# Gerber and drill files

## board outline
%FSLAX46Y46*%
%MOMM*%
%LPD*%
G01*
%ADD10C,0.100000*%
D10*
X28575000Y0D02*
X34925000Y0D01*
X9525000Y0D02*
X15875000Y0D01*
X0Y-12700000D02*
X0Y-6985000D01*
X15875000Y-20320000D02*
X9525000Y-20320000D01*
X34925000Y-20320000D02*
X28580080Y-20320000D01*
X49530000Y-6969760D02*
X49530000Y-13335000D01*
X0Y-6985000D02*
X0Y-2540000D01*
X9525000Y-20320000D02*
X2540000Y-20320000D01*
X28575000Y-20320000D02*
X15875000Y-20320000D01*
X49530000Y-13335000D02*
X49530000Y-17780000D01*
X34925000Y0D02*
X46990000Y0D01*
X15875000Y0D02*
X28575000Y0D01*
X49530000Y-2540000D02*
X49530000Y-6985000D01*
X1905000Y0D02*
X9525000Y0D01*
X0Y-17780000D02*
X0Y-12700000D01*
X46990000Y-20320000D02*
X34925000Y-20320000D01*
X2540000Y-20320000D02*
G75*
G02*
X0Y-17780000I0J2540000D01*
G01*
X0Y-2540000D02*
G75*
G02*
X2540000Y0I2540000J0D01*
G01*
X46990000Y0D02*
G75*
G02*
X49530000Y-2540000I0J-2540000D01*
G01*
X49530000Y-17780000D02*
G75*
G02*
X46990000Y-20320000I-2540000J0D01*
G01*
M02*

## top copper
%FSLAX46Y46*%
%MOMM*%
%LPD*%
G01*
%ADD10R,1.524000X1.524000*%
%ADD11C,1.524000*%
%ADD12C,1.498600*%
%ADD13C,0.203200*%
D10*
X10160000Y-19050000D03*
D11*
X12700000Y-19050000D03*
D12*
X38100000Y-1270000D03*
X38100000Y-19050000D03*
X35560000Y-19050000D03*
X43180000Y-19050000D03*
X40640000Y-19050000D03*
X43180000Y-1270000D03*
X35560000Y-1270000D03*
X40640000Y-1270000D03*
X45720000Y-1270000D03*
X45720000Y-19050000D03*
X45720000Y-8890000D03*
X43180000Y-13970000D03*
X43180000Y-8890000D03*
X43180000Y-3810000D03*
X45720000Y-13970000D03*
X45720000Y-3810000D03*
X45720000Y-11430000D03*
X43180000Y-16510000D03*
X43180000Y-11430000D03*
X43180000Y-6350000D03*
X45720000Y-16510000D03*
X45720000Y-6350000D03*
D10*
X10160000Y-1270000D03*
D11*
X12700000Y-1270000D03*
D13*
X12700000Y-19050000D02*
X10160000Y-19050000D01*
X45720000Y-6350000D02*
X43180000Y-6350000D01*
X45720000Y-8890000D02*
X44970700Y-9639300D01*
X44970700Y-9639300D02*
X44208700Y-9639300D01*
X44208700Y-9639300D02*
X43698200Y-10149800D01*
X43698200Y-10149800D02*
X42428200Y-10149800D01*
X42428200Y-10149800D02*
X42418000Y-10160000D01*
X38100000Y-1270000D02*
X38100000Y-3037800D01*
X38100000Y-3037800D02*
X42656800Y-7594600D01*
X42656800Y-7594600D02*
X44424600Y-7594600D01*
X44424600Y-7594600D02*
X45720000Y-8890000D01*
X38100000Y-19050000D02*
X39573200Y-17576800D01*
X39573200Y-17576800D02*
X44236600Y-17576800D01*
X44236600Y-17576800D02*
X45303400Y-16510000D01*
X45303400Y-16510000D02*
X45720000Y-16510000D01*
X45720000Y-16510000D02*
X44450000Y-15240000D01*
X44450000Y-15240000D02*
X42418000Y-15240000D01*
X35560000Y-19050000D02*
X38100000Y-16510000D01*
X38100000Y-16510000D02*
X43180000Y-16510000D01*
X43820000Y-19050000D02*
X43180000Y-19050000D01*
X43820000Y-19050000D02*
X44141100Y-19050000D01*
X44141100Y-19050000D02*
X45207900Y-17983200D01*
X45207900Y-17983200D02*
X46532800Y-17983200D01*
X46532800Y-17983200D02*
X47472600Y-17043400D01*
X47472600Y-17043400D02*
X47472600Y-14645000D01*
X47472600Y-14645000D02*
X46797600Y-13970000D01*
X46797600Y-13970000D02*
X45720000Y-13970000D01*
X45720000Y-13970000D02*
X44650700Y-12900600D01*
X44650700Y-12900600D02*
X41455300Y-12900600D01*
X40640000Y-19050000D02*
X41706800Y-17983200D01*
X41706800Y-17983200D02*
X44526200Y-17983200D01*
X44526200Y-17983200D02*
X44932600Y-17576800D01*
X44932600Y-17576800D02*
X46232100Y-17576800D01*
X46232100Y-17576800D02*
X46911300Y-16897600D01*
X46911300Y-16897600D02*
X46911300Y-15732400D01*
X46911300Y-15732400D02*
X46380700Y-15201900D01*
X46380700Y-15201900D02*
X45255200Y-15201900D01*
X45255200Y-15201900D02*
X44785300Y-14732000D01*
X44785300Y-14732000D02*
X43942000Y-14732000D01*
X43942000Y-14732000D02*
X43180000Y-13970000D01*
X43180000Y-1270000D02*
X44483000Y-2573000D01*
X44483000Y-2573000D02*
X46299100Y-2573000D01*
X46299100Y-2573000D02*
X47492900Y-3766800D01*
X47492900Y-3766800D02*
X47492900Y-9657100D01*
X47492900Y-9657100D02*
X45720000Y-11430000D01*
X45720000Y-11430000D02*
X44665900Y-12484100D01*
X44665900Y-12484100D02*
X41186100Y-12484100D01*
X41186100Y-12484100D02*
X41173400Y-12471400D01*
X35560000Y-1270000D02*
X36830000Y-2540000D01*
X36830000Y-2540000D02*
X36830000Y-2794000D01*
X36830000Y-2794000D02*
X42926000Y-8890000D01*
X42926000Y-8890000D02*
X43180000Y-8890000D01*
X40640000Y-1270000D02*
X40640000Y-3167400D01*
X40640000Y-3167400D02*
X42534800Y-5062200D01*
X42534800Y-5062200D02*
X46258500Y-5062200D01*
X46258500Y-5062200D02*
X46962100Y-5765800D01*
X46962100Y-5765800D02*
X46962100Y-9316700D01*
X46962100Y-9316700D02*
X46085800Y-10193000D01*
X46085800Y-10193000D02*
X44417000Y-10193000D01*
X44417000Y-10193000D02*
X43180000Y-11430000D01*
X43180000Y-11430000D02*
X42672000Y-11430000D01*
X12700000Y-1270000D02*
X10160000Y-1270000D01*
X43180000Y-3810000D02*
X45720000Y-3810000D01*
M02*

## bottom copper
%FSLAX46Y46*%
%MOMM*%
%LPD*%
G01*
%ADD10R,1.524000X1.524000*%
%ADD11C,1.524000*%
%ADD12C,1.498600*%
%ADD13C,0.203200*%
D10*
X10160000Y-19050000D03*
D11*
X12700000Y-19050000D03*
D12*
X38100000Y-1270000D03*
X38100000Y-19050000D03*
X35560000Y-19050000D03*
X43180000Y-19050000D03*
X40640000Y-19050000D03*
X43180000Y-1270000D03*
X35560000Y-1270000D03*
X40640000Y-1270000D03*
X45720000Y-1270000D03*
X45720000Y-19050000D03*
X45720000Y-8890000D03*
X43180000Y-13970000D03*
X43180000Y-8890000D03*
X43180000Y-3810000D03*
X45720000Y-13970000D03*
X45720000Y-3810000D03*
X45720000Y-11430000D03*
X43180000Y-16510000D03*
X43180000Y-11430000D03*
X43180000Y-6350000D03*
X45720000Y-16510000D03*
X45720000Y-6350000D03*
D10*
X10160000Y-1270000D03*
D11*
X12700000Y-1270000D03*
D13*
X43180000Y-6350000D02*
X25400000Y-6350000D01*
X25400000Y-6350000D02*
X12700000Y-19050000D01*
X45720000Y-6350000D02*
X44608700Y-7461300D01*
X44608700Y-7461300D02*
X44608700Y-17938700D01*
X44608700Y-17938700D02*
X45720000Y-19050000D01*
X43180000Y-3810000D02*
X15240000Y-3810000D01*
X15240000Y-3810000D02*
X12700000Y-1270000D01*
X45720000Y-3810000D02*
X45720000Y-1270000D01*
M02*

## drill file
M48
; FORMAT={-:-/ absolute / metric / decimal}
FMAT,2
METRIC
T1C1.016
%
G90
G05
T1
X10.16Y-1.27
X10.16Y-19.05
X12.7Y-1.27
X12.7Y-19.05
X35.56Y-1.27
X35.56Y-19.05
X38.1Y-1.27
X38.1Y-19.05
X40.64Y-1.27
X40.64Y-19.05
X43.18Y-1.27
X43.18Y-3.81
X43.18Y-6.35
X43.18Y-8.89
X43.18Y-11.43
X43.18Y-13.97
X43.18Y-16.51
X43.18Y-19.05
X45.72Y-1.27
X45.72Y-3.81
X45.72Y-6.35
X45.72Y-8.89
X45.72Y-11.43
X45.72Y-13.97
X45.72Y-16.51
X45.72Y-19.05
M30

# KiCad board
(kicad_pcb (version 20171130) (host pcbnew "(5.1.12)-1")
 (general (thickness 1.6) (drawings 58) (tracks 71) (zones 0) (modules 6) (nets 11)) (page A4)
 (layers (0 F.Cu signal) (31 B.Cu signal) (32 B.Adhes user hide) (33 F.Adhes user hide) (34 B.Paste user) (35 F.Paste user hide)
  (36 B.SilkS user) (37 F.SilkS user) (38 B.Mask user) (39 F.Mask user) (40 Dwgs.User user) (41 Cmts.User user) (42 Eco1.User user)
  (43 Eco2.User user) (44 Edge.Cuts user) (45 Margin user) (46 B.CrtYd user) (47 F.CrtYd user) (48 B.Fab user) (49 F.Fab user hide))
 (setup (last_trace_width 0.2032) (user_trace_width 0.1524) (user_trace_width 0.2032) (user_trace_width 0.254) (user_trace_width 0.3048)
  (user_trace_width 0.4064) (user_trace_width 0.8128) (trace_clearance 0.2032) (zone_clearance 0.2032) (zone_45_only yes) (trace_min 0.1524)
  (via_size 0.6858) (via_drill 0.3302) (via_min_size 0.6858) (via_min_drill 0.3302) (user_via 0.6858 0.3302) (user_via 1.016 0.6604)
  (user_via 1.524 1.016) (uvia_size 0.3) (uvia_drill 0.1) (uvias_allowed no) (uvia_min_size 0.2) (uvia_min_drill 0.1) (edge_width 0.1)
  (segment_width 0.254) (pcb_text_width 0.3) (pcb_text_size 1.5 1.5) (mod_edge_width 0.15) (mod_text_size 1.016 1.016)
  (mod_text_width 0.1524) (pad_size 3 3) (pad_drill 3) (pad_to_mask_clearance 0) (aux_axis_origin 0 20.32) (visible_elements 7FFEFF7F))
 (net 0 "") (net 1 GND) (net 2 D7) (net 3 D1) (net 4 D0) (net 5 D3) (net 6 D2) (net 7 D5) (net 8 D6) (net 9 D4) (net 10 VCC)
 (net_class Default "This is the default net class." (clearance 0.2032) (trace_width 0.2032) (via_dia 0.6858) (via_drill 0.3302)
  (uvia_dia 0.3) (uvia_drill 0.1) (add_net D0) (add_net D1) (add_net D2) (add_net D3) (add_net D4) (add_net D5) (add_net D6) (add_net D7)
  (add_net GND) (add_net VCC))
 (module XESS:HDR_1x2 (layer F.Cu) (at 11.43 19.05)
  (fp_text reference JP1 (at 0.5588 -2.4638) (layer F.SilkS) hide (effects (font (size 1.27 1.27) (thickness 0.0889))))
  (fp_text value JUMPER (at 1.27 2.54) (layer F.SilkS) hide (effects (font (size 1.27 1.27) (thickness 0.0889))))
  (pad 1 thru_hole rect (at -1.27 0) (size 1.524 1.524) (drill 1.016) (layers *.Cu *.Mask) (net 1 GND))
  (pad 2 thru_hole circle (at 1.27 0) (size 1.524 1.524) (drill 1.016) (layers *.Cu *.Mask) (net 1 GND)))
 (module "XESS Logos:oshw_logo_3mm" (layer B.Cu) (at 10.16 10.16 270)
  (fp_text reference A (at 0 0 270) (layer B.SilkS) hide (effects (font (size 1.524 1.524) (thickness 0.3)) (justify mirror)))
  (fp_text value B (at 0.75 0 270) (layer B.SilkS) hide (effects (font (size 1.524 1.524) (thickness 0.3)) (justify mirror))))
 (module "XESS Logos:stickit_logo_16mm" (layer B.Cu) (at 17.145 12.065 270)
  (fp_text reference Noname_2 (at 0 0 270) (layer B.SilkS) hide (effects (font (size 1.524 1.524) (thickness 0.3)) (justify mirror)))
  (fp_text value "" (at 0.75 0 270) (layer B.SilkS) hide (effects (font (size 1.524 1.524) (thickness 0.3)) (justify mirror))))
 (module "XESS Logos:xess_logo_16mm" (layer B.Cu) (at 31.75 10.16 270)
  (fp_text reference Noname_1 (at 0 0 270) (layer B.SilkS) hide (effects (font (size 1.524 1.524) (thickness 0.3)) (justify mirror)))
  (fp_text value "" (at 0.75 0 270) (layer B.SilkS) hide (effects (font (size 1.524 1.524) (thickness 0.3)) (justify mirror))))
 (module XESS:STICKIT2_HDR (layer F.Cu) (at 44.45 10.16 180)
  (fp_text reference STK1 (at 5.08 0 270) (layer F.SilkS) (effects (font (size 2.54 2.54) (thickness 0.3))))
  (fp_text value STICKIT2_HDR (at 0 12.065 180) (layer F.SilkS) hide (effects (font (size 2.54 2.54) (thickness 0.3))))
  (pad D7 thru_hole circle (at 6.35 8.89 270) (size 1.4986 1.4986) (drill 1.016) (layers *.Cu *.Mask) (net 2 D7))
  (pad D1 thru_hole circle (at 6.35 -8.89 270) (size 1.4986 1.4986) (drill 1.016) (layers *.Cu *.Mask) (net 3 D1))
  (pad D0 thru_hole circle (at 8.89 -8.89 180) (size 1.4986 1.4986) (drill 1.016) (layers *.Cu *.Mask) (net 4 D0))
  (pad D3 thru_hole circle (at 1.27 -8.89 270) (size 1.4986 1.4986) (drill 1.016) (layers *.Cu *.Mask) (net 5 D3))
  (pad D2 thru_hole circle (at 3.81 -8.89 270) (size 1.4986 1.4986) (drill 1.016) (layers *.Cu *.Mask) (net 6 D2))
  (pad D5 thru_hole circle (at 1.27 8.89 270) (size 1.4986 1.4986) (drill 1.016) (layers *.Cu *.Mask) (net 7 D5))
  (pad D6 thru_hole circle (at 8.89 8.89 270) (size 1.4986 1.4986) (drill 1.016) (layers *.Cu *.Mask) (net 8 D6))
  (pad D4 thru_hole circle (at 3.81 8.89 270) (size 1.4986 1.4986) (drill 1.016) (layers *.Cu *.Mask) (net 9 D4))
  (pad VCC thru_hole circle (at -1.27 8.89 270) (size 1.4986 1.4986) (drill 1.016) (layers *.Cu *.Mask) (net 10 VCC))
  (pad GND thru_hole circle (at -1.27 -8.89 270) (size 1.4986 1.4986) (drill 1.016) (layers *.Cu *.Mask) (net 1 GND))
  (pad D7 thru_hole circle (at -1.27 1.27 270) (size 1.4986 1.4986) (drill 1.016) (layers *.Cu *.Mask) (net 2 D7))
  (pad D2 thru_hole circle (at 1.27 -3.81 270) (size 1.4986 1.4986) (drill 1.016) (layers *.Cu *.Mask) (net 6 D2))
  (pad D6 thru_hole circle (at 1.27 1.27 270) (size 1.4986 1.4986) (drill 1.016) (layers *.Cu *.Mask) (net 8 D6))
  (pad VCC thru_hole circle (at 1.27 6.35 270) (size 1.4986 1.4986) (drill 1.016) (layers *.Cu *.Mask) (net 10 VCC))
  (pad D3 thru_hole circle (at -1.27 -3.81 270) (size 1.4986 1.4986) (drill 1.016) (layers *.Cu *.Mask) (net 5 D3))
  (pad VCC thru_hole circle (at -1.27 6.35 270) (size 1.4986 1.4986) (drill 1.016) (layers *.Cu *.Mask) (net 10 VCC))
  (pad D5 thru_hole circle (at -1.27 -1.27 270) (size 1.4986 1.4986) (drill 1.016) (layers *.Cu *.Mask) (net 7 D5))
  (pad D0 thru_hole circle (at 1.27 -6.35 180) (size 1.4986 1.4986) (drill 1.016) (layers *.Cu *.Mask) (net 4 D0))
  (pad D4 thru_hole circle (at 1.27 -1.27 270) (size 1.4986 1.4986) (drill 1.016) (layers *.Cu *.Mask) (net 9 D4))
  (pad GND thru_hole circle (at 1.27 3.81 270) (size 1.4986 1.4986) (drill 1.016) (layers *.Cu *.Mask) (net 1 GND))
  (pad D1 thru_hole circle (at -1.27 -6.35 270) (size 1.4986 1.4986) (drill 1.016) (layers *.Cu *.Mask) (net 3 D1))
  (pad GND thru_hole circle (at -1.27 3.81 270) (size 1.4986 1.4986) (drill 1.016) (layers *.Cu *.Mask) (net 1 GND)))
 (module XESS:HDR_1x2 (layer F.Cu) (at 11.43 1.27)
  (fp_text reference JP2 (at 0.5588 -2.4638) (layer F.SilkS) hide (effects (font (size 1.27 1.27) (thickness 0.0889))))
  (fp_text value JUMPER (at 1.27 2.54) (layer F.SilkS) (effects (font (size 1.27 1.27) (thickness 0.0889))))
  (pad 1 thru_hole rect (at -1.27 0) (size 1.524 1.524) (drill 1.016) (layers *.Cu *.Mask) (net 10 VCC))
  (pad 2 thru_hole circle (at 1.27 0) (size 1.524 1.524) (drill 1.016) (layers *.Cu *.Mask) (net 10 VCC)))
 (gr_line (start 28.575 0) (end 34.925 0) (layer Edge.Cuts) (width 0.1))
 (gr_line (start 9.525 0) (end 15.875 0) (layer Edge.Cuts) (width 0.1))
 (gr_line (start 0 12.7) (end 0 6.985) (layer Edge.Cuts) (width 0.1))
 (gr_line (start 15.875 20.32) (end 9.525 20.32) (layer Edge.Cuts) (width 0.1))
 (gr_line (start 34.925 20.32) (end 28.58008 20.32) (layer Edge.Cuts) (width 0.1))
 (gr_line (start 49.53 6.96976) (end 49.53 13.335) (layer Edge.Cuts) (width 0.1))
 (gr_line (start 0 6.985) (end 0 2.54) (angle 90) (layer Edge.Cuts) (width 0.1))
 (gr_line (start 9.525 20.32) (end 2.54 20.32) (angle 90) (layer Edge.Cuts) (width 0.1))
 (gr_line (start 28.575 20.32) (end 15.875 20.32) (angle 90) (layer Edge.Cuts) (width 0.1))
 (gr_line (start 49.53 13.335) (end 49.53 17.78) (angle 90) (layer Edge.Cuts) (width 0.1))
 (gr_line (start 34.925 0) (end 46.99 0) (angle 90) (layer Edge.Cuts) (width 0.1))
 (gr_line (start 15.875 0) (end 28.575 0) (angle 90) (layer Edge.Cuts) (width 0.1))
 (gr_line (start 49.53 2.54) (end 49.53 6.985) (angle 90) (layer Edge.Cuts) (width 0.1))
 (gr_line (start 1.905 0) (end 9.525 0) (angle 90) (layer Edge.Cuts) (width 0.1))
 (gr_line (start 0 17.78) (end 0 12.7) (angle 90) (layer Edge.Cuts) (width 0.1))
 (gr_line (start 46.99 20.32) (end 34.925 20.32) (angle 90) (layer Edge.Cuts) (width 0.1))
 (gr_arc (start 2.54 17.78) (end 2.54 20.32) (angle 90) (layer Edge.Cuts) (width 0.1))
 (gr_arc (start 2.54 2.54) (end 0 2.54) (angle 90) (layer Edge.Cuts) (width 0.1))
 (gr_arc (start 46.99 2.54) (end 46.99 0) (angle 90) (layer Edge.Cuts) (width 0.1))
 (gr_arc (start 46.99 17.78) (end 49.53 17.78) (angle 90) (layer Edge.Cuts) (width 0.1))
 (segment (start 12.7 19.05) (end 10.16 19.05) (width 0.2032) (layer F.Cu) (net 1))
 (segment (start 43.18 6.35) (end 25.4 6.35) (width 0.2032) (layer B.Cu) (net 1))
 (segment (start 25.4 6.35) (end 12.7 19.05) (width 0.2032) (layer B.Cu) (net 1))
 (segment (start 45.72 6.35) (end 44.6087 7.4613) (width 0.2032) (layer B.Cu) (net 1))
 (segment (start 44.6087 7.4613) (end 44.6087 17.9387) (width 0.2032) (layer B.Cu) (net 1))
 (segment (start 44.6087 17.9387) (end 45.72 19.05) (width 0.2032) (layer B.Cu) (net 1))
 (segment (start 45.72 6.35) (end 43.18 6.35) (width 0.2032) (layer F.Cu) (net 1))
 (segment (start 45.72 8.89) (end 44.9707 9.6393) (width 0.2032) (layer F.Cu) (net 2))
 (segment (start 44.9707 9.6393) (end 44.2087 9.6393) (width 0.2032) (layer F.Cu) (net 2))
 (segment (start 44.2087 9.6393) (end 43.6982 10.1498) (width 0.2032) (layer F.Cu) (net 2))
 (segment (start 43.6982 10.1498) (end 42.4282 10.1498) (width 0.2032) (layer F.Cu) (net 2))
 (segment (start 42.4282 10.1498) (end 42.418 10.16) (width 0.2032) (layer F.Cu) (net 2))
 (segment (start 38.1 1.27) (end 38.1 3.0378) (width 0.2032) (layer F.Cu) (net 2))
 (segment (start 38.1 3.0378) (end 42.6568 7.5946) (width 0.2032) (layer F.Cu) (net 2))
 (segment (start 42.6568 7.5946) (end 44.4246 7.5946) (width 0.2032) (layer F.Cu) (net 2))
 (segment (start 44.4246 7.5946) (end 45.72 8.89) (width 0.2032) (layer F.Cu) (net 2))
 (segment (start 38.1 19.05) (end 39.5732 17.5768) (width 0.2032) (layer F.Cu) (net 3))
 (segment (start 39.5732 17.5768) (end 44.2366 17.5768) (width 0.2032) (layer F.Cu) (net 3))
 (segment (start 44.2366 17.5768) (end 45.3034 16.51) (width 0.2032) (layer F.Cu) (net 3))
 (segment (start 45.3034 16.51) (end 45.72 16.51) (width 0.2032) (layer F.Cu) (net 3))
 (segment (start 45.72 16.51) (end 44.45 15.24) (width 0.2032) (layer F.Cu) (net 3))
 (segment (start 44.45 15.24) (end 42.418 15.24) (width 0.2032) (layer F.Cu) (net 3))
 (segment (start 35.56 19.05) (end 38.1 16.51) (width 0.2032) (layer F.Cu) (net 4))
 (segment (start 38.1 16.51) (end 43.18 16.51) (width 0.2032) (layer F.Cu) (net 4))
 (segment (start 43.82 19.05) (end 43.18 19.05) (width 0.2032) (layer F.Cu) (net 5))
 (segment (start 43.82 19.05) (end 44.1411 19.05) (width 0.2032) (layer F.Cu) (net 5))
 (segment (start 44.1411 19.05) (end 45.2079 17.9832) (width 0.2032) (layer F.Cu) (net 5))
 (segment (start 45.2079 17.9832) (end 46.5328 17.9832) (width 0.2032) (layer F.Cu) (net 5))
 (segment (start 46.5328 17.9832) (end 47.4726 17.0434) (width 0.2032) (layer F.Cu) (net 5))
 (segment (start 47.4726 17.0434) (end 47.4726 14.645) (width 0.2032) (layer F.Cu) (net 5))
 (segment (start 47.4726 14.645) (end 46.7976 13.97) (width 0.2032) (layer F.Cu) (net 5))
 (segment (start 46.7976 13.97) (end 45.72 13.97) (width 0.2032) (layer F.Cu) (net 5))
 (segment (start 45.72 13.97) (end 44.6507 12.9006) (width 0.2032) (layer F.Cu) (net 5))
 (segment (start 44.6507 12.9006) (end 41.4553 12.9006) (width 0.2032) (layer F.Cu) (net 5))
 (segment (start 40.64 19.05) (end 41.7068 17.9832) (width 0.2032) (layer F.Cu) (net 6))
 (segment (start 41.7068 17.9832) (end 44.5262 17.9832) (width 0.2032) (layer F.Cu) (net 6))
 (segment (start 44.5262 17.9832) (end 44.9326 17.5768) (width 0.2032) (layer F.Cu) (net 6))
 (segment (start 44.9326 17.5768) (end 46.2321 17.5768) (width 0.2032) (layer F.Cu) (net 6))
 (segment (start 46.2321 17.5768) (end 46.9113 16.8976) (width 0.2032) (layer F.Cu) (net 6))
 (segment (start 46.9113 16.8976) (end 46.9113 15.7324) (width 0.2032) (layer F.Cu) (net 6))
 (segment (start 46.9113 15.7324) (end 46.3807 15.2019) (width 0.2032) (layer F.Cu) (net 6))
 (segment (start 46.3807 15.2019) (end 45.2552 15.2019) (width 0.2032) (layer F.Cu) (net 6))
 (segment (start 45.2552 15.2019) (end 44.7853 14.732) (width 0.2032) (layer F.Cu) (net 6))
 (segment (start 44.7853 14.732) (end 43.942 14.732) (width 0.2032) (layer F.Cu) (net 6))
 (segment (start 43.942 14.732) (end 43.18 13.97) (width 0.2032) (layer F.Cu) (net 6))
 (segment (start 43.18 1.27) (end 44.483 2.573) (width 0.2032) (layer F.Cu) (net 7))
 (segment (start 44.483 2.573) (end 46.2991 2.573) (width 0.2032) (layer F.Cu) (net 7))
 (segment (start 46.2991 2.573) (end 47.4929 3.7668) (width 0.2032) (layer F.Cu) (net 7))
 (segment (start 47.4929 3.7668) (end 47.4929 9.6571) (width 0.2032) (layer F.Cu) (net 7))
 (segment (start 47.4929 9.6571) (end 45.72 11.43) (width 0.2032) (layer F.Cu) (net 7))
 (segment (start 45.72 11.43) (end 44.6659 12.4841) (width 0.2032) (layer F.Cu) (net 7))
 (segment (start 44.6659 12.4841) (end 41.1861 12.4841) (width 0.2032) (layer F.Cu) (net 7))
 (segment (start 41.1861 12.4841) (end 41.1734 12.4714) (width 0.2032) (layer F.Cu) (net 7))
 (segment (start 35.56 1.27) (end 36.83 2.54) (width 0.2032) (layer F.Cu) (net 8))
 (segment (start 36.83 2.54) (end 36.83 2.794) (width 0.2032) (layer F.Cu) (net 8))
 (segment (start 36.83 2.794) (end 42.926 8.89) (width 0.2032) (layer F.Cu) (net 8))
 (segment (start 42.926 8.89) (end 43.18 8.89) (width 0.2032) (layer F.Cu) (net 8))
 (segment (start 40.64 1.27) (end 40.64 3.1674) (width 0.2032) (layer F.Cu) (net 9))
 (segment (start 40.64 3.1674) (end 42.5348 5.0622) (width 0.2032) (layer F.Cu) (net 9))
 (segment (start 42.5348 5.0622) (end 46.2585 5.0622) (width 0.2032) (layer F.Cu) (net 9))
 (segment (start 46.2585 5.0622) (end 46.9621 5.7658) (width 0.2032) (layer F.Cu) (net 9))
 (segment (start 46.9621 5.7658) (end 46.9621 9.3167) (width 0.2032) (layer F.Cu) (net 9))
 (segment (start 46.9621 9.3167) (end 46.0858 10.193) (width 0.2032) (layer F.Cu) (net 9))
 (segment (start 46.0858 10.193) (end 44.417 10.193) (width 0.2032) (layer F.Cu) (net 9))
 (segment (start 44.417 10.193) (end 43.18 11.43) (width 0.2032) (layer F.Cu) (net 9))
 (segment (start 43.18 11.43) (end 42.672 11.43) (width 0.2032) (layer F.Cu) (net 9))
 (segment (start 12.7 1.27) (end 10.16 1.27) (width 0.2032) (layer F.Cu) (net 10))
 (segment (start 43.18 3.81) (end 15.24 3.81) (width 0.2032) (layer B.Cu) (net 10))
 (segment (start 15.24 3.81) (end 12.7 1.27) (width 0.2032) (layer B.Cu) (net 10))
 (segment (start 43.18 3.81) (end 45.72 3.81) (width 0.2032) (layer F.Cu) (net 10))
 (segment (start 45.72 3.81) (end 45.72 1.27) (width 0.2032) (layer B.Cu) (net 10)))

